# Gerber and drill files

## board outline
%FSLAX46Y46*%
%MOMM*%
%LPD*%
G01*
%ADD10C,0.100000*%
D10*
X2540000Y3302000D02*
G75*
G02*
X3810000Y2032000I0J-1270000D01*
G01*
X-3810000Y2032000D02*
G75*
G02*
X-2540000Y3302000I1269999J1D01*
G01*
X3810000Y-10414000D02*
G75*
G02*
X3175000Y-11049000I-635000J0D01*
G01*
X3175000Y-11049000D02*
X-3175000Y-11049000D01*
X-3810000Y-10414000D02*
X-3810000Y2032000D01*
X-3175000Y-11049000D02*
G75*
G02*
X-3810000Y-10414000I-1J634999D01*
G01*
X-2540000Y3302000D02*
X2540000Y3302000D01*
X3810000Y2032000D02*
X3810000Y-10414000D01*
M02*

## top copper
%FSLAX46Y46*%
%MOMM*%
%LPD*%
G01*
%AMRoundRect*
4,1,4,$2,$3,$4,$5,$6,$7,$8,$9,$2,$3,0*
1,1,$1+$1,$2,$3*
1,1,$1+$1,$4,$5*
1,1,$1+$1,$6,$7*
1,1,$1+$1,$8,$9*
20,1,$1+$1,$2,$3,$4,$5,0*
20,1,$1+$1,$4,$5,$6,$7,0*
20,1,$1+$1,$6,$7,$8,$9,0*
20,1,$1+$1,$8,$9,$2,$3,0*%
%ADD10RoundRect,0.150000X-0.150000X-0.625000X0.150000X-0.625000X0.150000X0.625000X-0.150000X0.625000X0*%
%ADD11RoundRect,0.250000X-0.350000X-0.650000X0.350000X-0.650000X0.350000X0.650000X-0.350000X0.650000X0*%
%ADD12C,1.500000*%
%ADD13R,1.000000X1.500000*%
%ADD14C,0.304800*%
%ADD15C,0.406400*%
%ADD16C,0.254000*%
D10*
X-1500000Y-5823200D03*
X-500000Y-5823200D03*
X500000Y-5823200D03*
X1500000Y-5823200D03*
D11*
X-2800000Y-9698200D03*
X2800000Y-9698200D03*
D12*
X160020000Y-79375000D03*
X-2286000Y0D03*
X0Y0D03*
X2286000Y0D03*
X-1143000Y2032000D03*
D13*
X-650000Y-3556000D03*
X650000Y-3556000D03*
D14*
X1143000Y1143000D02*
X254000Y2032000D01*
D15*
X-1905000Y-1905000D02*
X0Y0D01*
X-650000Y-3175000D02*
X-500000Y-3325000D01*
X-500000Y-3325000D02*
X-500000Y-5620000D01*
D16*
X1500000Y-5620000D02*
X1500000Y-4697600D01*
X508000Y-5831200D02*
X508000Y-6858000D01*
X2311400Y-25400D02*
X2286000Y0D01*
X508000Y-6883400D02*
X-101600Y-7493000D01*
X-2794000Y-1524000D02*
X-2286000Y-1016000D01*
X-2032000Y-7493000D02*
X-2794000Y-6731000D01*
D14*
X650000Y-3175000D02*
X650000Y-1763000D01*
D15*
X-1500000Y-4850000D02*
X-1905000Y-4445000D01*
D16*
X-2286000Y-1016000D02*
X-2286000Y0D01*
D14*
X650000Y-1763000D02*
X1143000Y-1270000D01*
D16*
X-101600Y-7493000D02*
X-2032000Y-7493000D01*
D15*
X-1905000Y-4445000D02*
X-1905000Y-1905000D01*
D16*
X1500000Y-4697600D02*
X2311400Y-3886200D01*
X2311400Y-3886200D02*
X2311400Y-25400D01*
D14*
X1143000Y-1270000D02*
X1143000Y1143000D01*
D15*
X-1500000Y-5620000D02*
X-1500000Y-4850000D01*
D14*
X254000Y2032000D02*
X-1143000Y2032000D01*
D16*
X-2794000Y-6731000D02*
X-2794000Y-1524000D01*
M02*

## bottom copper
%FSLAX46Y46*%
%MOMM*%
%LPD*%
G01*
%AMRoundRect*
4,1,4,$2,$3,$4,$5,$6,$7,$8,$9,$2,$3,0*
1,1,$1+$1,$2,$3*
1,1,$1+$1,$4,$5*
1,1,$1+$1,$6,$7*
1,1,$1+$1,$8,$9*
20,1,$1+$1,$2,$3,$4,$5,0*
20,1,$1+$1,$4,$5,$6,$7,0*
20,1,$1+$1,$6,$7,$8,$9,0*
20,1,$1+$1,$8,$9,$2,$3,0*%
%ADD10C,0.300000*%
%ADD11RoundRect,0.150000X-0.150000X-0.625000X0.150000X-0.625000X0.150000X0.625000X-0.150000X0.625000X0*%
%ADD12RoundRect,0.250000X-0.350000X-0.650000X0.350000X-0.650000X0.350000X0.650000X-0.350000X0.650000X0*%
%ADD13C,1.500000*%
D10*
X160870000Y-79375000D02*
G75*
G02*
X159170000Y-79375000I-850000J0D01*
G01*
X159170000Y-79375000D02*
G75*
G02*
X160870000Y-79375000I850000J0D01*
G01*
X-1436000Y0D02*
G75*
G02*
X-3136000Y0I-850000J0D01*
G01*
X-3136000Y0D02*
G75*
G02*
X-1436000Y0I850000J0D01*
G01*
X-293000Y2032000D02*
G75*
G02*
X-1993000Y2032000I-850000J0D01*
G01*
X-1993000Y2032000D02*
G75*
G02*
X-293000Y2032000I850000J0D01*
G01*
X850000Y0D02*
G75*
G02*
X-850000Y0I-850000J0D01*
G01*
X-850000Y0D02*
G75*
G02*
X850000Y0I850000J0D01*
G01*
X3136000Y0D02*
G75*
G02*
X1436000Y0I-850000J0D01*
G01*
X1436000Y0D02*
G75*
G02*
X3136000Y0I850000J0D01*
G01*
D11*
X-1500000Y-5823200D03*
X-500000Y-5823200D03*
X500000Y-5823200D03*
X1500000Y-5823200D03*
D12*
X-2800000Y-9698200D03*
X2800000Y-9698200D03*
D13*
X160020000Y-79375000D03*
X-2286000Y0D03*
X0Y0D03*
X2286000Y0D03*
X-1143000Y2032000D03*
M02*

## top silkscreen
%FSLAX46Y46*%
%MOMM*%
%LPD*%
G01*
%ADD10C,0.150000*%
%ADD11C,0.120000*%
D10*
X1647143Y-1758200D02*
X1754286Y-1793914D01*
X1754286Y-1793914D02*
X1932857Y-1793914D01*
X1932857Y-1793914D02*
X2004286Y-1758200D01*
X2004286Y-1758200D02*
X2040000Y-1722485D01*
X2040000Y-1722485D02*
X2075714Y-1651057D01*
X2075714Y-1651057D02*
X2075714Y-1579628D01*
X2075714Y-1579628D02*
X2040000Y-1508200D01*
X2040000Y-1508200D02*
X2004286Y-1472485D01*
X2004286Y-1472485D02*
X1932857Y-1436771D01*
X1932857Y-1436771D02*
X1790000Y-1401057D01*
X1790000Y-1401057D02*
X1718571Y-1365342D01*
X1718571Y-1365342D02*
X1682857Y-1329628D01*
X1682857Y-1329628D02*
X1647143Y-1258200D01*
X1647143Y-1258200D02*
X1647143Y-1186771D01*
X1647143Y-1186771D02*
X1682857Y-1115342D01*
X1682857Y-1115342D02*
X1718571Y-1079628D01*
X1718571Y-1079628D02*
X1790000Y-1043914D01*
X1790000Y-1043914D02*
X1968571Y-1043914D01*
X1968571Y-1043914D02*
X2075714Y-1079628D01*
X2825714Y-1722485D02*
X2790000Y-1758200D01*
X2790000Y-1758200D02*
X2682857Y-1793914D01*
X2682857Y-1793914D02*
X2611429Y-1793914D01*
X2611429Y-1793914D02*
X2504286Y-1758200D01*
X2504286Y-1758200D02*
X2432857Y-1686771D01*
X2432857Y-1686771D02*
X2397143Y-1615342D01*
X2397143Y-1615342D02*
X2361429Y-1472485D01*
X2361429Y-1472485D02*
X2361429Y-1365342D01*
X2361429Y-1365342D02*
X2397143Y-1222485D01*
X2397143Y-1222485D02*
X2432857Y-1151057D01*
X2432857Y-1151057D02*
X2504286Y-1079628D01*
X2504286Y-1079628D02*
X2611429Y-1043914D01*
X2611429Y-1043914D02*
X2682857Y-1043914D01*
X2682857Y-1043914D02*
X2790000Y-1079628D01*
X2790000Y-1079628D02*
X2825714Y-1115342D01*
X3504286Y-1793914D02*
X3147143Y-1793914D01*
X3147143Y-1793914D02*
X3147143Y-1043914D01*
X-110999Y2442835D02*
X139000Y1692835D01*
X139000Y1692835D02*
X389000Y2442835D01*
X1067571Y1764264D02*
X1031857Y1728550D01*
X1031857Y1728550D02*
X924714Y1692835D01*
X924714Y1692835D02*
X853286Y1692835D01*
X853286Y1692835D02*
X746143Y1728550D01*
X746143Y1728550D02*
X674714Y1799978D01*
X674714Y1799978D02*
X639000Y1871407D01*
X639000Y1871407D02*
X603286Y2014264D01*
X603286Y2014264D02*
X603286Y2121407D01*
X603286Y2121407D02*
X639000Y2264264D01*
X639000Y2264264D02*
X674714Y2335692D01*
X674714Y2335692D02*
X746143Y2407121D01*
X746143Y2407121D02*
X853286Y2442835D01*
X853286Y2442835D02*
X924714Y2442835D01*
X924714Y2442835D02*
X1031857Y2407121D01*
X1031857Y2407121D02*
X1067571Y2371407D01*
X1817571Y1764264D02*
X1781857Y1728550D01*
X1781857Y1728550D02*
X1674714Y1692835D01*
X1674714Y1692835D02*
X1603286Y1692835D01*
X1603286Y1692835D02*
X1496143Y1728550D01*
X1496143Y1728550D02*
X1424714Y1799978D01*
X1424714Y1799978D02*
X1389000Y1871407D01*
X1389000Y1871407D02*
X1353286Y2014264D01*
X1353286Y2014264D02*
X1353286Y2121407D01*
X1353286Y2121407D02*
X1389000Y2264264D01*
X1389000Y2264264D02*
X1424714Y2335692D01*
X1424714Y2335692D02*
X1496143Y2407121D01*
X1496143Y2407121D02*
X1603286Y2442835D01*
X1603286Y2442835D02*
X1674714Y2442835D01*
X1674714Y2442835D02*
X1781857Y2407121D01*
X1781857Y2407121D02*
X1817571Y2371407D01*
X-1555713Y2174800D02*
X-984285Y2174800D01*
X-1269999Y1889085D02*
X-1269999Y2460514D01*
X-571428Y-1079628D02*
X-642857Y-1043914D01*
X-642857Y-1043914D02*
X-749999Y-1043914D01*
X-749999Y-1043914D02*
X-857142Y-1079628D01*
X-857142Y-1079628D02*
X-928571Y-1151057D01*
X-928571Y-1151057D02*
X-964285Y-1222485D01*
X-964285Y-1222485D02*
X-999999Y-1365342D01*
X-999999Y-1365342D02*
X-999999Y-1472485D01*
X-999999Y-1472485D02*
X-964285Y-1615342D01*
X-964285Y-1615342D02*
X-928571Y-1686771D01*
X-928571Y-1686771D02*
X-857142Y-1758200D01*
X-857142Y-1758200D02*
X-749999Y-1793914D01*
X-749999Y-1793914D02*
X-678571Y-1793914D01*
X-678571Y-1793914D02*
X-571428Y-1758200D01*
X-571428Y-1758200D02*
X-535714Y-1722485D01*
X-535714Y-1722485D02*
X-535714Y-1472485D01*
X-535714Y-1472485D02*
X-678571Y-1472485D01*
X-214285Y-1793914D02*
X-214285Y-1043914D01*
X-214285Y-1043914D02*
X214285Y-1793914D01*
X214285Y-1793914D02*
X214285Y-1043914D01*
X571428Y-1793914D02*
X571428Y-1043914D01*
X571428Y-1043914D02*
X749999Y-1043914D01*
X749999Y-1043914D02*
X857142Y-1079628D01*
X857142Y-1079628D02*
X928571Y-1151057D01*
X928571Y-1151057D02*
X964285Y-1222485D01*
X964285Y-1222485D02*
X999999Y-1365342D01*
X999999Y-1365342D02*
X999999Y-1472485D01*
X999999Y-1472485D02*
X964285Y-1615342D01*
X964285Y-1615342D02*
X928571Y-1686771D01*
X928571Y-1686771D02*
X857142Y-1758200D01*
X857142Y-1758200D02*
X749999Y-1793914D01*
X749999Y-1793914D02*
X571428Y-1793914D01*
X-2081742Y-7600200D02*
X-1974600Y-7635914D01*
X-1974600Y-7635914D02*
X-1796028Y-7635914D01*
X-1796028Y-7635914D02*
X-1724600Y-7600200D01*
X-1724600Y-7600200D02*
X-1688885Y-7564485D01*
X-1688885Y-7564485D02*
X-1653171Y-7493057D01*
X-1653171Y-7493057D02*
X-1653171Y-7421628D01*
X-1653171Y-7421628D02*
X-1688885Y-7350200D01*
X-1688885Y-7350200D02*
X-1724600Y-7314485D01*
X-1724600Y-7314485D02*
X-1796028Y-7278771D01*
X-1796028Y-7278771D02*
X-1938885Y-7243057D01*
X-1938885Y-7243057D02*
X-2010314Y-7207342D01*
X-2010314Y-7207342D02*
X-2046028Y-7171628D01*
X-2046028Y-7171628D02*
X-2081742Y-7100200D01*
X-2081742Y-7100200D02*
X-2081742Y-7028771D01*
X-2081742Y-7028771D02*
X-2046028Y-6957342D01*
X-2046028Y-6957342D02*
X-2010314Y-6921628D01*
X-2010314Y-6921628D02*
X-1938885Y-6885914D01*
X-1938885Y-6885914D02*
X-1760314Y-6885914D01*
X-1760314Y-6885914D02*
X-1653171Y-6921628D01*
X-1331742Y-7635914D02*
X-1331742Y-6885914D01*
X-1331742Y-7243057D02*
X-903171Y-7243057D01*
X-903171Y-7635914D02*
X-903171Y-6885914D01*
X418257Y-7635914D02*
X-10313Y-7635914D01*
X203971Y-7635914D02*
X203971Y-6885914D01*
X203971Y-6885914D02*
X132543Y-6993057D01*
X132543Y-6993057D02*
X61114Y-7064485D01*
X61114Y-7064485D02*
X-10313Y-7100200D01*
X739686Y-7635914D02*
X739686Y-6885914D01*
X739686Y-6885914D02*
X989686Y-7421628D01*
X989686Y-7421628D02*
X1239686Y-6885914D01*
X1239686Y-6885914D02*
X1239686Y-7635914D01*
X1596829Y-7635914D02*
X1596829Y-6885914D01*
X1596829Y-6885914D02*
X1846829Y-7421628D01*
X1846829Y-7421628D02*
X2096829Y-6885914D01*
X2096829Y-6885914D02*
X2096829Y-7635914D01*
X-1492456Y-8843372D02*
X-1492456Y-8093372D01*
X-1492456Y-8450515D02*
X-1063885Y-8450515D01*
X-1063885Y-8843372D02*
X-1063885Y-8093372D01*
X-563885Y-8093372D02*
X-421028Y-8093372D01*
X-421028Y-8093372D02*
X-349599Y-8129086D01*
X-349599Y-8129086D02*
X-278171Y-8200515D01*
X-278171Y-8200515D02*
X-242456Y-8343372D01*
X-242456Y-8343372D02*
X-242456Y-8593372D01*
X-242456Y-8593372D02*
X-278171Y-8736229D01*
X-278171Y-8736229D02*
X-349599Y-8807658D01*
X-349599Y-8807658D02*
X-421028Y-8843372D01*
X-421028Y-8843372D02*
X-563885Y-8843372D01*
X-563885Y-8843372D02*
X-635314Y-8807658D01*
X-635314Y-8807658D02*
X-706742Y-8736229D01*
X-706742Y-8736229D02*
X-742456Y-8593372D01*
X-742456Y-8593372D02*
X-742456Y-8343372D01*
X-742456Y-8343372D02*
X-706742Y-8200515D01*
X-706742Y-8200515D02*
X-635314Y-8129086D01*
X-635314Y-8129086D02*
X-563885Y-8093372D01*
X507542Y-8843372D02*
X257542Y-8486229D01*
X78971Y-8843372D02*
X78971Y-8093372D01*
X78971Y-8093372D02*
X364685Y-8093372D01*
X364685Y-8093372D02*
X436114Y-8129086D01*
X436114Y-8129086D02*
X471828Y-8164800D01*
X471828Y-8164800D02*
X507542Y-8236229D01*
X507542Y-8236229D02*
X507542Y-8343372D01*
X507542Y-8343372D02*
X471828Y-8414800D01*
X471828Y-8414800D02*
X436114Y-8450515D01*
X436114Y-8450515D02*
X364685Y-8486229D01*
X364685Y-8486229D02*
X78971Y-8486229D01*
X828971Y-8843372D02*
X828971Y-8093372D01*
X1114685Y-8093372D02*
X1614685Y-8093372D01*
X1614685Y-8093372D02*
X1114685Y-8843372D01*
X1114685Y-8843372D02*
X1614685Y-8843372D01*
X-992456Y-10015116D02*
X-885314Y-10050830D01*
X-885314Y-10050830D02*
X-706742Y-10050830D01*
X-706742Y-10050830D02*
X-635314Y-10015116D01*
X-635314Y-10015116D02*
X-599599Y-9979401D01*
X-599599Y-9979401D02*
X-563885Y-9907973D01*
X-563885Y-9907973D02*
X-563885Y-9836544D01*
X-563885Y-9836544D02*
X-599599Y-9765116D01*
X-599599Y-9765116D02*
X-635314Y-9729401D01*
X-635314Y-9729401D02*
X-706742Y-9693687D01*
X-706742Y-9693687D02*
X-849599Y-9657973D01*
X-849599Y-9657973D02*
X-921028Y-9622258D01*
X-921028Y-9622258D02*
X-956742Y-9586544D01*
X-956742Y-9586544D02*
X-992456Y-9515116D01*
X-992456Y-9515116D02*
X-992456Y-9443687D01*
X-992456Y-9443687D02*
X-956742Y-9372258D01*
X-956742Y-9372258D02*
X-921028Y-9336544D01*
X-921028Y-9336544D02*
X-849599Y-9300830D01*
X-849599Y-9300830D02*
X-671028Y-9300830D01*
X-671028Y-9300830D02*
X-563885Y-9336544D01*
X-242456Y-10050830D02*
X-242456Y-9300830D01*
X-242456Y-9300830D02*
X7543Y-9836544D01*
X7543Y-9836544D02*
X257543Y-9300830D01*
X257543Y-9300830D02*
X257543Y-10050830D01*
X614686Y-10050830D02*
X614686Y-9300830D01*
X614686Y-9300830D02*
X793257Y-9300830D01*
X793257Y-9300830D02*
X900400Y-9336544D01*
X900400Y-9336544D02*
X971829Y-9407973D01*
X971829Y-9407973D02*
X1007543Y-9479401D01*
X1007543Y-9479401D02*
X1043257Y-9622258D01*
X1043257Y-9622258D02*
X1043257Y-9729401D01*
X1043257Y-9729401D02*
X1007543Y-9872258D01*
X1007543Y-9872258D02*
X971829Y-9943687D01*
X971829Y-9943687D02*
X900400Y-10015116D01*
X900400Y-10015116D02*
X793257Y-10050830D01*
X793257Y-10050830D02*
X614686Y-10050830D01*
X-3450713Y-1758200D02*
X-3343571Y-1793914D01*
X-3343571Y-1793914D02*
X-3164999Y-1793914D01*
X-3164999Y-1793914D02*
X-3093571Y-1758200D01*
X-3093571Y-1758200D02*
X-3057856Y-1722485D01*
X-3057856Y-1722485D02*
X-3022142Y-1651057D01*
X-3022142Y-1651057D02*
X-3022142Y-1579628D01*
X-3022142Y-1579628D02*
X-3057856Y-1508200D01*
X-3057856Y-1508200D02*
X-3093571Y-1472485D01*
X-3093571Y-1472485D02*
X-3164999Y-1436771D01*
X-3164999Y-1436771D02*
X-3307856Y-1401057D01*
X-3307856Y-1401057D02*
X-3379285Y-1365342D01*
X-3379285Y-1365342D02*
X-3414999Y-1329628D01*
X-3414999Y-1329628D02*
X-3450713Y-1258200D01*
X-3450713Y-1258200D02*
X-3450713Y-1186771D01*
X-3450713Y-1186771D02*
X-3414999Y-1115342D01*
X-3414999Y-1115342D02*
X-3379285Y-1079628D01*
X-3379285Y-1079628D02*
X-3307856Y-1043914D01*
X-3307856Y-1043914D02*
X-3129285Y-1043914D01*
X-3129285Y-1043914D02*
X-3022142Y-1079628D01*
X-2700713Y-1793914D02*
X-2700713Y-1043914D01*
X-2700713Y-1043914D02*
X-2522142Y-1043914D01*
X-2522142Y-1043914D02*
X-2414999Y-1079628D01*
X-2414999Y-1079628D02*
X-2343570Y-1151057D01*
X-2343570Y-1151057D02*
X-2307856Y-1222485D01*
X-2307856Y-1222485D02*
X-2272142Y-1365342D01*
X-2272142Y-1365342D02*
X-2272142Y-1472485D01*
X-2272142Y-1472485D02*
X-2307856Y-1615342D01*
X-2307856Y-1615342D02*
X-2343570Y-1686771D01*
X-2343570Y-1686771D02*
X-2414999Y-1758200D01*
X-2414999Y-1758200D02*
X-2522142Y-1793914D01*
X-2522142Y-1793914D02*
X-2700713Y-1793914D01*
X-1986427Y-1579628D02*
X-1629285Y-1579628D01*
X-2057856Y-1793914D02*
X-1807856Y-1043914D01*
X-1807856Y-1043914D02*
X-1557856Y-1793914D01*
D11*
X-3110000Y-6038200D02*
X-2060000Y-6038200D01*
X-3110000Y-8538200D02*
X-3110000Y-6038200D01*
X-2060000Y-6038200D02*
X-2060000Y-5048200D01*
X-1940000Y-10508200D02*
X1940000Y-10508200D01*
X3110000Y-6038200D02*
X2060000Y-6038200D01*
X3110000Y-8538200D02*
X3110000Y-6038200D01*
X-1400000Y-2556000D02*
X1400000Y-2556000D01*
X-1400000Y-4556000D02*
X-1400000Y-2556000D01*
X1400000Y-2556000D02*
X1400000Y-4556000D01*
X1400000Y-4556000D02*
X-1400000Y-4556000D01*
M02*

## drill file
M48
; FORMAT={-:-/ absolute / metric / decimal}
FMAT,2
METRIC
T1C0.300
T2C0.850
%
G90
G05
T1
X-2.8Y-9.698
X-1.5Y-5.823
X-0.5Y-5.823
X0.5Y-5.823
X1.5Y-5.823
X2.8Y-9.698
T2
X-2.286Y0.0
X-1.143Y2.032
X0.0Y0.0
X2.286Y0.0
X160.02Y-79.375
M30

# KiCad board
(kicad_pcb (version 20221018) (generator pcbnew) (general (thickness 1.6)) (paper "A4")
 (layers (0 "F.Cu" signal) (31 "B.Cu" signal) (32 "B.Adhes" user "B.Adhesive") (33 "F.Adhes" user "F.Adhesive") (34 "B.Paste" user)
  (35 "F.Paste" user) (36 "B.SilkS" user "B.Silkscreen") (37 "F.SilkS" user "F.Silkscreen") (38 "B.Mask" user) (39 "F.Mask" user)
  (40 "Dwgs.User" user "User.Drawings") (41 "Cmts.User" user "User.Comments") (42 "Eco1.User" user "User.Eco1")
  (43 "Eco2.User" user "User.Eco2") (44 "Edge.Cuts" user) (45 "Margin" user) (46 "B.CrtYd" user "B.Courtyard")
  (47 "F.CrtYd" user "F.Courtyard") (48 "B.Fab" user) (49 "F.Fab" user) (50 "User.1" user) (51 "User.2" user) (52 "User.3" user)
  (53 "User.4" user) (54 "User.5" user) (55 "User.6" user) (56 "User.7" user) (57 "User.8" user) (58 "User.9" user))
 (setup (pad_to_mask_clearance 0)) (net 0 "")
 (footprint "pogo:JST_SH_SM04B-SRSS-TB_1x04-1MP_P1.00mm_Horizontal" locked (layer "F.Cu") (at 0 7.8232)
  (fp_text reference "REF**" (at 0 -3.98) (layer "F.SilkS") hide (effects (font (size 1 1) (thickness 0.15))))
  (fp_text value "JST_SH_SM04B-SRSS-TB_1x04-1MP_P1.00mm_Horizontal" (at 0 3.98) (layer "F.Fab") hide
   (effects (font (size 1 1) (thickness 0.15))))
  (fp_line (start -3.11 -1.785) (end -2.06 -1.785) (stroke (width 0.12) (type solid)) (layer "F.SilkS"))
  (fp_line (start -3.11 0.715) (end -3.11 -1.785) (stroke (width 0.12) (type solid)) (layer "F.SilkS"))
  (fp_line (start -2.06 -1.785) (end -2.06 -2.775) (stroke (width 0.12) (type solid)) (layer "F.SilkS"))
  (fp_line (start -1.94 2.685) (end 1.94 2.685) (stroke (width 0.12) (type solid)) (layer "F.SilkS"))
  (fp_line (start 3.11 -1.785) (end 2.06 -1.785) (stroke (width 0.12) (type solid)) (layer "F.SilkS"))
  (fp_line (start 3.11 0.715) (end 3.11 -1.785) (stroke (width 0.12) (type solid)) (layer "F.SilkS"))
  (pad "1" thru_hole roundrect locked (at -1.5 -2) (size 0.6 1.55) (drill 0.3) (layers "*.Cu" "F.Paste" "F.Mask") (roundrect_rratio 0.25))
  (pad "2" thru_hole roundrect locked (at -0.5 -2) (size 0.6 1.55) (drill 0.3) (layers "*.Cu" "F.Paste" "F.Mask") (roundrect_rratio 0.25))
  (pad "3" thru_hole roundrect locked (at 0.5 -2) (size 0.6 1.55) (drill 0.3) (layers "*.Cu" "F.Paste" "F.Mask") (roundrect_rratio 0.25))
  (pad "4" thru_hole roundrect locked (at 1.5 -2) (size 0.6 1.55) (drill 0.3) (layers "*.Cu" "F.Paste" "F.Mask") (roundrect_rratio 0.25))
  (pad "MP" thru_hole roundrect locked (at -2.8 1.875) (size 1.2 1.8) (drill 0.3) (layers "*.Cu" "F.Paste" "F.Mask")
   (roundrect_rratio 0.2083333333))
  (pad "MP" thru_hole roundrect locked (at 2.8 1.875) (size 1.2 1.8) (drill 0.3) (layers "*.Cu" "F.Paste" "F.Mask")
   (roundrect_rratio 0.2083333333)))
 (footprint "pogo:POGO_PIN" (layer "F.Cu") (at 160.02 79.375)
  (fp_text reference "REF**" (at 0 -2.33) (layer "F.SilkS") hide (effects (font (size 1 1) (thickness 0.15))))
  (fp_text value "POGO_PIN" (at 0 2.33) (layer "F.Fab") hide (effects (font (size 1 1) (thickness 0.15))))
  (fp_circle (center 0 0) (end 0.85 0) (stroke (width 0.3) (type solid)) (fill none) (layer "B.Cu"))
  (pad "1" thru_hole circle (at 0 0) (size 1.5 1.5) (drill 0.85) (layers "*.Cu" "*.Mask")))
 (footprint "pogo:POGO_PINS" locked (layer "F.Cu") (at 0 0)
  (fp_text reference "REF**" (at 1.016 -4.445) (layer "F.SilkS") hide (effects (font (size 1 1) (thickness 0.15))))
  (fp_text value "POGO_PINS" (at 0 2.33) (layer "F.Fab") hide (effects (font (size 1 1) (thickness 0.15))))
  (fp_circle (center -2.286 0) (end -1.436 0) (stroke (width 0.3) (type solid)) (fill none) (layer "B.Cu"))
  (fp_circle (center -1.143 -2.032) (end -0.293 -2.032) (stroke (width 0.3) (type solid)) (fill none) (layer "B.Cu"))
  (fp_circle (center 0 0) (end 0.85 0) (stroke (width 0.3) (type solid)) (fill none) (layer "B.Cu"))
  (fp_circle (center 2.286 0) (end 3.136 0) (stroke (width 0.3) (type solid)) (fill none) (layer "B.Cu"))
  (pad "1" thru_hole circle locked (at -2.286 0) (size 1.5 1.5) (drill 0.85) (layers "*.Cu" "*.Mask"))
  (pad "2" thru_hole circle locked (at 0 0) (size 1.5 1.5) (drill 0.85) (layers "*.Cu" "*.Mask"))
  (pad "3" thru_hole circle locked (at 2.286 0) (size 1.5 1.5) (drill 0.85) (layers "*.Cu" "*.Mask"))
  (pad "4" thru_hole circle locked (at -1.143 -2.032) (size 1.5 1.5) (drill 0.85) (layers "*.Cu" "*.Mask")))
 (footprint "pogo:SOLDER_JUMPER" (layer "F.Cu") (at 0 3.556)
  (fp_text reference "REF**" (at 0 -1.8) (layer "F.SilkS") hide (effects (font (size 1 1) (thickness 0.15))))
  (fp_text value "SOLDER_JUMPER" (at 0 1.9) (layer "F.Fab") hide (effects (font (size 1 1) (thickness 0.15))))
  (fp_line (start -1.4 -1) (end 1.4 -1) (stroke (width 0.12) (type solid)) (layer "F.SilkS"))
  (fp_line (start -1.4 1) (end -1.4 -1) (stroke (width 0.12) (type solid)) (layer "F.SilkS"))
  (fp_line (start 1.4 -1) (end 1.4 1) (stroke (width 0.12) (type solid)) (layer "F.SilkS"))
  (fp_line (start 1.4 1) (end -1.4 1) (stroke (width 0.12) (type solid)) (layer "F.SilkS"))
  (pad "1" smd rect (at -0.65 0) (size 1 1.5) (layers "F.Cu" "F.Mask"))
  (pad "2" smd rect (at 0.65 0) (size 1 1.5) (layers "F.Cu" "F.Mask")))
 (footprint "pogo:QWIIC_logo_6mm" (layer "B.Cu") (at 0.040263 4.7302 180)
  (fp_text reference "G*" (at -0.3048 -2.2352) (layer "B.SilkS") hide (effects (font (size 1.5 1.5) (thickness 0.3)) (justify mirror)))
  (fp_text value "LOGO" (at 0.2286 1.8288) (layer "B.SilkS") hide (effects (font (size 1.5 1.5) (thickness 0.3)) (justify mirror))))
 (gr_arc (start 2.54 -3.302) (mid 3.438026 -2.930026) (end 3.81 -2.032) (stroke (width 0.1) (type default)) (layer "Edge.Cuts"))
 (gr_arc (start -3.81 -2.032) (mid -3.438026 -2.930026) (end -2.54 -3.302) (stroke (width 0.1) (type default)) (layer "Edge.Cuts"))
 (gr_arc (start 3.81 10.414) (mid 3.624013 10.863013) (end 3.175 11.049) (stroke (width 0.1) (type default)) (layer "Edge.Cuts"))
 (gr_line (start 3.175 11.049) (end -3.175 11.049) (stroke (width 0.1) (type default)) (layer "Edge.Cuts"))
 (gr_line (start -3.81 10.414) (end -3.81 -2.032) (stroke (width 0.1) (type default)) (layer "Edge.Cuts"))
 (gr_arc (start -3.175 11.049) (mid -3.624013 10.863013) (end -3.81 10.414) (stroke (width 0.1) (type default)) (layer "Edge.Cuts"))
 (gr_line (start -2.54 -3.302) (end 2.54 -3.302) (stroke (width 0.1) (type default)) (layer "Edge.Cuts"))
 (gr_line (start 3.81 -2.032) (end 3.81 10.414) (stroke (width 0.1) (type default)) (layer "Edge.Cuts"))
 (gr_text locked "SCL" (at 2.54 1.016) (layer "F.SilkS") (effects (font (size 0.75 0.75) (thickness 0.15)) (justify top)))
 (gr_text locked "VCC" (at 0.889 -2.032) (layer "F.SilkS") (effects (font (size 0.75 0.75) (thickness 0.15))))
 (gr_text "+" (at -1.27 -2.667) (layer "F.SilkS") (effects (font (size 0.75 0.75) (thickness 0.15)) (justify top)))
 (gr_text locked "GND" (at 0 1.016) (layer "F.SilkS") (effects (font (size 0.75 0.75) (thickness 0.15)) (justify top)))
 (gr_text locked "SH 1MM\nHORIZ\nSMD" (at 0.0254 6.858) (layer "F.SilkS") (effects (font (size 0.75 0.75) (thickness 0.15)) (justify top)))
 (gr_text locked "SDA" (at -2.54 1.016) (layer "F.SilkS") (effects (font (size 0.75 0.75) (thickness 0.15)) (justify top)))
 (segment (start 1.143 -1.143) (end 0.254 -2.032) (width 0.3048) (layer "F.Cu") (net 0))
 (segment (start -1.905 1.905) (end 0 0) (width 0.4064) (layer "F.Cu") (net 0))
 (segment (start -0.65 3.175) (end -0.5 3.325) (width 0.4064) (layer "F.Cu") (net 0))
 (segment (start -0.5 3.325) (end -0.5 5.62) (width 0.4064) (layer "F.Cu") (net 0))
 (segment (start 1.5 5.62) (end 1.5 4.6976) (width 0.254) (layer "F.Cu") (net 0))
 (segment (start 0.508 5.8312) (end 0.508 6.858) (width 0.254) (layer "F.Cu") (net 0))
 (segment (start 2.3114 0.0254) (end 2.286 0) (width 0.254) (layer "F.Cu") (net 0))
 (segment (start 0.508 6.8834) (end -0.1016 7.493) (width 0.254) (layer "F.Cu") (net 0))
 (segment (start -2.794 1.524) (end -2.286 1.016) (width 0.254) (layer "F.Cu") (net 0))
 (segment (start -2.032 7.493) (end -2.794 6.731) (width 0.254) (layer "F.Cu") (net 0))
 (segment (start 0.65 3.175) (end 0.65 1.763) (width 0.3048) (layer "F.Cu") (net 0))
 (segment (start -1.5 4.85) (end -1.905 4.445) (width 0.4064) (layer "F.Cu") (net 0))
 (segment (start -2.286 1.016) (end -2.286 0) (width 0.254) (layer "F.Cu") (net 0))
 (segment (start 0.65 1.763) (end 1.143 1.27) (width 0.3048) (layer "F.Cu") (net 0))
 (segment (start -0.1016 7.493) (end -2.032 7.493) (width 0.254) (layer "F.Cu") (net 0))
 (segment (start -1.905 4.445) (end -1.905 1.905) (width 0.4064) (layer "F.Cu") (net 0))
 (segment (start 1.5 4.6976) (end 2.3114 3.8862) (width 0.254) (layer "F.Cu") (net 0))
 (segment (start 2.3114 3.8862) (end 2.3114 0.0254) (width 0.254) (layer "F.Cu") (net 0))
 (segment (start 1.143 1.27) (end 1.143 -1.143) (width 0.3048) (layer "F.Cu") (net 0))
 (segment (start -1.5 5.62) (end -1.5 4.85) (width 0.4064) (layer "F.Cu") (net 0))
 (segment (start 0.254 -2.032) (end -1.143 -2.032) (width 0.3048) (layer "F.Cu") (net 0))
 (segment (start -2.794 6.731) (end -2.794 1.524) (width 0.254) (layer "F.Cu") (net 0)))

